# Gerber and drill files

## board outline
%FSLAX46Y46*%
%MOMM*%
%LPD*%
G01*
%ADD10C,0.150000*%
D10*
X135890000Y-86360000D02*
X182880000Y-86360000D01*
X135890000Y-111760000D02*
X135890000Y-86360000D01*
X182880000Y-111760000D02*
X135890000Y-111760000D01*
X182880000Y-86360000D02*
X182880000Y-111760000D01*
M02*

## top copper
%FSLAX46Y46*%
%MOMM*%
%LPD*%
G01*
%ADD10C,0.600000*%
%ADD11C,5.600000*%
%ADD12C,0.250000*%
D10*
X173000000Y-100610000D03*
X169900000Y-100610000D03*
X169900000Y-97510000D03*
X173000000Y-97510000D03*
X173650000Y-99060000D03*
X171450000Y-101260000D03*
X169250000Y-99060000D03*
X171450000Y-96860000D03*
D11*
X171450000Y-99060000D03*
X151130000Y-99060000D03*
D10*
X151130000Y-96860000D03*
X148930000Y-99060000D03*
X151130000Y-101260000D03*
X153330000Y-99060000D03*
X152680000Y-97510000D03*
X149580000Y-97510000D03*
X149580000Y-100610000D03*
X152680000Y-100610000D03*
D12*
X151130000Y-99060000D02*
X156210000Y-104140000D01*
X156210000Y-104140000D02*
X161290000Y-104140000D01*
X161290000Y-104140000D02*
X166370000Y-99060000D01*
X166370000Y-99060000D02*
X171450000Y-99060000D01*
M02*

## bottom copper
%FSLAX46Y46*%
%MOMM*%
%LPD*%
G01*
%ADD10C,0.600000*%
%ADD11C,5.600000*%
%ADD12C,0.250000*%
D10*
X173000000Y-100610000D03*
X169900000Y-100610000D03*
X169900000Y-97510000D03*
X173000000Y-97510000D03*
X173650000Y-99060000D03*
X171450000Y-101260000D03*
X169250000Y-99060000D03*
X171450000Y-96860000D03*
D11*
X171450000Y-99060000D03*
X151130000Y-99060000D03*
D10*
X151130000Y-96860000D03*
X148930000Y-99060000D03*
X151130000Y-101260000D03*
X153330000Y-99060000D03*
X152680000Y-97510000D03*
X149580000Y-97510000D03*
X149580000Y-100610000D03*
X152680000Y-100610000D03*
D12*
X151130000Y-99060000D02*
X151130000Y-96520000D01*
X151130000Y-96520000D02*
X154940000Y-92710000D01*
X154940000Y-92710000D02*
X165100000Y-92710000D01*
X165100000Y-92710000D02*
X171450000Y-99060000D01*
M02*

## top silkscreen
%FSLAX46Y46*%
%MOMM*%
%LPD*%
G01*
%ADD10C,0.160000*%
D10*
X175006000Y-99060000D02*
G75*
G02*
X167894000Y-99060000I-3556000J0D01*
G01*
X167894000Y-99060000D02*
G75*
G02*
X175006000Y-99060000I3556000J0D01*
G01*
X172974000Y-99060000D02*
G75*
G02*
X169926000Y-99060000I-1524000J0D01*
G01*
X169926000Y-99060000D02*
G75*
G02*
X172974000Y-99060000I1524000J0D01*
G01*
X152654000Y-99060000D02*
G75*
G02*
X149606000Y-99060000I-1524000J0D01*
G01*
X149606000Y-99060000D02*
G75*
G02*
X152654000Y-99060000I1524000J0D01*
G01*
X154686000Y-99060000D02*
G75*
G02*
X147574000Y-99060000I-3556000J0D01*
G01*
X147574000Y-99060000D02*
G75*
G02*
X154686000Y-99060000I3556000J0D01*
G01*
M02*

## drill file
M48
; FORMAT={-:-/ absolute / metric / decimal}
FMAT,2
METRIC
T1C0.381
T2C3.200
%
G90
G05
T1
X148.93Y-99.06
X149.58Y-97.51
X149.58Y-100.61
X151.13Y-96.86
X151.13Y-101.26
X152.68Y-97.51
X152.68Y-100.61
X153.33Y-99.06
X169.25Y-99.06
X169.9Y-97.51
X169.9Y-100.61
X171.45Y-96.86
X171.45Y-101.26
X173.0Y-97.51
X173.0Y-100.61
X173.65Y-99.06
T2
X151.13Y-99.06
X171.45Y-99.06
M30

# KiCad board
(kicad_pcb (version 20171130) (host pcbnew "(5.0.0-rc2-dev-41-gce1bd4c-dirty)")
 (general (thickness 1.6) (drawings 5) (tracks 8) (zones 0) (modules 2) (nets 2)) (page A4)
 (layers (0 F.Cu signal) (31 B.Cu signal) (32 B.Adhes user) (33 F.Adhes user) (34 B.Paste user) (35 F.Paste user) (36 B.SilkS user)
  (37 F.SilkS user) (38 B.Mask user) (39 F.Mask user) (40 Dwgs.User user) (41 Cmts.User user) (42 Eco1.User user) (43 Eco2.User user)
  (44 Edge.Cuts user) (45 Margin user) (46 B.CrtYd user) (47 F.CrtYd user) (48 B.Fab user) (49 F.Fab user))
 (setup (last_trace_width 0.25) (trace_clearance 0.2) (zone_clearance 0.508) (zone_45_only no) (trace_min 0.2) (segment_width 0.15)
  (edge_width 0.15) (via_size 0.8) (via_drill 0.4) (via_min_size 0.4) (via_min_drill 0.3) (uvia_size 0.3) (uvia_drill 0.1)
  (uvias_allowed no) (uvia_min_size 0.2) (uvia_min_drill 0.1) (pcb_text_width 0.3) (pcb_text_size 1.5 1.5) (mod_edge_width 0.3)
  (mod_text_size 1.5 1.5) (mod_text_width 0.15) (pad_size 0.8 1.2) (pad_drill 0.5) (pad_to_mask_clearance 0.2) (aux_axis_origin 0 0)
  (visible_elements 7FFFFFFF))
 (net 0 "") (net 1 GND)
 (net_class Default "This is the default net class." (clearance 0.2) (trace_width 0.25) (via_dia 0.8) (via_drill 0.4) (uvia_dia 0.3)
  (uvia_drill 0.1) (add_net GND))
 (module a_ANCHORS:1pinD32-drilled (layer F.Cu) (at 171.45 99.06)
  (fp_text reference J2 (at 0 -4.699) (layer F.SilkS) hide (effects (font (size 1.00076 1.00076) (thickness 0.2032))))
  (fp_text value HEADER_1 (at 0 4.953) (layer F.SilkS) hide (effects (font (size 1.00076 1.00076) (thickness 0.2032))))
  (fp_circle (center 0 0) (end 0 3.556) (layer F.SilkS) (width 0.16))
  (fp_circle (center 0 0) (end 0 1.524) (layer F.SilkS) (width 0.16))
  (pad 1 thru_hole circle (at 1.55 1.55) (size 0.6 0.6) (drill 0.381) (layers *.Cu *.Mask) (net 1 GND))
  (pad 1 thru_hole circle (at -1.55 1.55) (size 0.6 0.6) (drill 0.381) (layers *.Cu *.Mask) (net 1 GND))
  (pad 1 thru_hole circle (at -1.55 -1.55) (size 0.6 0.6) (drill 0.381) (layers *.Cu *.Mask) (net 1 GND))
  (pad 1 thru_hole circle (at 1.55 -1.55) (size 0.6 0.6) (drill 0.381) (layers *.Cu *.Mask) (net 1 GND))
  (pad 1 thru_hole circle (at 2.2 0) (size 0.6 0.6) (drill 0.381) (layers *.Cu *.Mask) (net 1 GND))
  (pad 1 thru_hole circle (at 0 2.2) (size 0.6 0.6) (drill 0.381) (layers *.Cu *.Mask) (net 1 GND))
  (pad 1 thru_hole circle (at -2.2 0) (size 0.6 0.6) (drill 0.381) (layers *.Cu *.Mask) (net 1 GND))
  (pad 1 thru_hole circle (at 0 -2.2) (size 0.6 0.6) (drill 0.381) (layers *.Cu *.Mask) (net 1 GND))
  (pad 1 thru_hole circle (at 0 0) (size 5.6 5.6) (drill 3.2004) (layers *.Cu *.Mask) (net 1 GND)))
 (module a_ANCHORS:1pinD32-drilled (layer F.Cu) (at 151.13 99.06)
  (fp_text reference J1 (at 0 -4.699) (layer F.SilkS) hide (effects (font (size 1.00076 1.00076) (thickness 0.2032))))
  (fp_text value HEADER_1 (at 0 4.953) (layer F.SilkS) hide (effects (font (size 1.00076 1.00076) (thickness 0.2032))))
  (fp_circle (center 0 0) (end 0 1.524) (layer F.SilkS) (width 0.16))
  (fp_circle (center 0 0) (end 0 3.556) (layer F.SilkS) (width 0.16))
  (pad 1 thru_hole circle (at 0 0) (size 5.6 5.6) (drill 3.2004) (layers *.Cu *.Mask) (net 1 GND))
  (pad 1 thru_hole circle (at 0 -2.2) (size 0.6 0.6) (drill 0.381) (layers *.Cu *.Mask) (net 1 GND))
  (pad 1 thru_hole circle (at -2.2 0) (size 0.6 0.6) (drill 0.381) (layers *.Cu *.Mask) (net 1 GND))
  (pad 1 thru_hole circle (at 0 2.2) (size 0.6 0.6) (drill 0.381) (layers *.Cu *.Mask) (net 1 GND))
  (pad 1 thru_hole circle (at 2.2 0) (size 0.6 0.6) (drill 0.381) (layers *.Cu *.Mask) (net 1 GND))
  (pad 1 thru_hole circle (at 1.55 -1.55) (size 0.6 0.6) (drill 0.381) (layers *.Cu *.Mask) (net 1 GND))
  (pad 1 thru_hole circle (at -1.55 -1.55) (size 0.6 0.6) (drill 0.381) (layers *.Cu *.Mask) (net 1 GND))
  (pad 1 thru_hole circle (at -1.55 1.55) (size 0.6 0.6) (drill 0.381) (layers *.Cu *.Mask) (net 1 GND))
  (pad 1 thru_hole circle (at 1.55 1.55) (size 0.6 0.6) (drill 0.381) (layers *.Cu *.Mask) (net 1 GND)))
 (gr_line (start 135.89 86.36) (end 182.88 86.36) (angle 90) (layer Edge.Cuts) (width 0.15))
 (gr_line (start 135.89 111.76) (end 135.89 86.36) (angle 90) (layer Edge.Cuts) (width 0.15))
 (gr_line (start 182.88 111.76) (end 135.89 111.76) (angle 90) (layer Edge.Cuts) (width 0.15))
 (gr_line (start 182.88 86.36) (end 182.88 111.76) (angle 90) (layer Edge.Cuts) (width 0.15))
 (segment (start 151.13 99.06) (end 156.21 104.14) (width 0.25) (layer F.Cu) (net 1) (status 400000))
 (segment (start 156.21 104.14) (end 161.29 104.14) (width 0.25) (layer F.Cu) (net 1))
 (segment (start 161.29 104.14) (end 166.37 99.06) (width 0.25) (layer F.Cu) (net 1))
 (segment (start 166.37 99.06) (end 171.45 99.06) (width 0.25) (layer F.Cu) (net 1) (status 800000))
 (segment (start 151.13 99.06) (end 151.13 96.52) (width 0.25) (layer B.Cu) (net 1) (status 400000))
 (segment (start 151.13 96.52) (end 154.94 92.71) (width 0.25) (layer B.Cu) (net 1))
 (segment (start 154.94 92.71) (end 165.1 92.71) (width 0.25) (layer B.Cu) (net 1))
 (segment (start 165.1 92.71) (end 171.45 99.06) (width 0.25) (layer B.Cu) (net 1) (status 800000)))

